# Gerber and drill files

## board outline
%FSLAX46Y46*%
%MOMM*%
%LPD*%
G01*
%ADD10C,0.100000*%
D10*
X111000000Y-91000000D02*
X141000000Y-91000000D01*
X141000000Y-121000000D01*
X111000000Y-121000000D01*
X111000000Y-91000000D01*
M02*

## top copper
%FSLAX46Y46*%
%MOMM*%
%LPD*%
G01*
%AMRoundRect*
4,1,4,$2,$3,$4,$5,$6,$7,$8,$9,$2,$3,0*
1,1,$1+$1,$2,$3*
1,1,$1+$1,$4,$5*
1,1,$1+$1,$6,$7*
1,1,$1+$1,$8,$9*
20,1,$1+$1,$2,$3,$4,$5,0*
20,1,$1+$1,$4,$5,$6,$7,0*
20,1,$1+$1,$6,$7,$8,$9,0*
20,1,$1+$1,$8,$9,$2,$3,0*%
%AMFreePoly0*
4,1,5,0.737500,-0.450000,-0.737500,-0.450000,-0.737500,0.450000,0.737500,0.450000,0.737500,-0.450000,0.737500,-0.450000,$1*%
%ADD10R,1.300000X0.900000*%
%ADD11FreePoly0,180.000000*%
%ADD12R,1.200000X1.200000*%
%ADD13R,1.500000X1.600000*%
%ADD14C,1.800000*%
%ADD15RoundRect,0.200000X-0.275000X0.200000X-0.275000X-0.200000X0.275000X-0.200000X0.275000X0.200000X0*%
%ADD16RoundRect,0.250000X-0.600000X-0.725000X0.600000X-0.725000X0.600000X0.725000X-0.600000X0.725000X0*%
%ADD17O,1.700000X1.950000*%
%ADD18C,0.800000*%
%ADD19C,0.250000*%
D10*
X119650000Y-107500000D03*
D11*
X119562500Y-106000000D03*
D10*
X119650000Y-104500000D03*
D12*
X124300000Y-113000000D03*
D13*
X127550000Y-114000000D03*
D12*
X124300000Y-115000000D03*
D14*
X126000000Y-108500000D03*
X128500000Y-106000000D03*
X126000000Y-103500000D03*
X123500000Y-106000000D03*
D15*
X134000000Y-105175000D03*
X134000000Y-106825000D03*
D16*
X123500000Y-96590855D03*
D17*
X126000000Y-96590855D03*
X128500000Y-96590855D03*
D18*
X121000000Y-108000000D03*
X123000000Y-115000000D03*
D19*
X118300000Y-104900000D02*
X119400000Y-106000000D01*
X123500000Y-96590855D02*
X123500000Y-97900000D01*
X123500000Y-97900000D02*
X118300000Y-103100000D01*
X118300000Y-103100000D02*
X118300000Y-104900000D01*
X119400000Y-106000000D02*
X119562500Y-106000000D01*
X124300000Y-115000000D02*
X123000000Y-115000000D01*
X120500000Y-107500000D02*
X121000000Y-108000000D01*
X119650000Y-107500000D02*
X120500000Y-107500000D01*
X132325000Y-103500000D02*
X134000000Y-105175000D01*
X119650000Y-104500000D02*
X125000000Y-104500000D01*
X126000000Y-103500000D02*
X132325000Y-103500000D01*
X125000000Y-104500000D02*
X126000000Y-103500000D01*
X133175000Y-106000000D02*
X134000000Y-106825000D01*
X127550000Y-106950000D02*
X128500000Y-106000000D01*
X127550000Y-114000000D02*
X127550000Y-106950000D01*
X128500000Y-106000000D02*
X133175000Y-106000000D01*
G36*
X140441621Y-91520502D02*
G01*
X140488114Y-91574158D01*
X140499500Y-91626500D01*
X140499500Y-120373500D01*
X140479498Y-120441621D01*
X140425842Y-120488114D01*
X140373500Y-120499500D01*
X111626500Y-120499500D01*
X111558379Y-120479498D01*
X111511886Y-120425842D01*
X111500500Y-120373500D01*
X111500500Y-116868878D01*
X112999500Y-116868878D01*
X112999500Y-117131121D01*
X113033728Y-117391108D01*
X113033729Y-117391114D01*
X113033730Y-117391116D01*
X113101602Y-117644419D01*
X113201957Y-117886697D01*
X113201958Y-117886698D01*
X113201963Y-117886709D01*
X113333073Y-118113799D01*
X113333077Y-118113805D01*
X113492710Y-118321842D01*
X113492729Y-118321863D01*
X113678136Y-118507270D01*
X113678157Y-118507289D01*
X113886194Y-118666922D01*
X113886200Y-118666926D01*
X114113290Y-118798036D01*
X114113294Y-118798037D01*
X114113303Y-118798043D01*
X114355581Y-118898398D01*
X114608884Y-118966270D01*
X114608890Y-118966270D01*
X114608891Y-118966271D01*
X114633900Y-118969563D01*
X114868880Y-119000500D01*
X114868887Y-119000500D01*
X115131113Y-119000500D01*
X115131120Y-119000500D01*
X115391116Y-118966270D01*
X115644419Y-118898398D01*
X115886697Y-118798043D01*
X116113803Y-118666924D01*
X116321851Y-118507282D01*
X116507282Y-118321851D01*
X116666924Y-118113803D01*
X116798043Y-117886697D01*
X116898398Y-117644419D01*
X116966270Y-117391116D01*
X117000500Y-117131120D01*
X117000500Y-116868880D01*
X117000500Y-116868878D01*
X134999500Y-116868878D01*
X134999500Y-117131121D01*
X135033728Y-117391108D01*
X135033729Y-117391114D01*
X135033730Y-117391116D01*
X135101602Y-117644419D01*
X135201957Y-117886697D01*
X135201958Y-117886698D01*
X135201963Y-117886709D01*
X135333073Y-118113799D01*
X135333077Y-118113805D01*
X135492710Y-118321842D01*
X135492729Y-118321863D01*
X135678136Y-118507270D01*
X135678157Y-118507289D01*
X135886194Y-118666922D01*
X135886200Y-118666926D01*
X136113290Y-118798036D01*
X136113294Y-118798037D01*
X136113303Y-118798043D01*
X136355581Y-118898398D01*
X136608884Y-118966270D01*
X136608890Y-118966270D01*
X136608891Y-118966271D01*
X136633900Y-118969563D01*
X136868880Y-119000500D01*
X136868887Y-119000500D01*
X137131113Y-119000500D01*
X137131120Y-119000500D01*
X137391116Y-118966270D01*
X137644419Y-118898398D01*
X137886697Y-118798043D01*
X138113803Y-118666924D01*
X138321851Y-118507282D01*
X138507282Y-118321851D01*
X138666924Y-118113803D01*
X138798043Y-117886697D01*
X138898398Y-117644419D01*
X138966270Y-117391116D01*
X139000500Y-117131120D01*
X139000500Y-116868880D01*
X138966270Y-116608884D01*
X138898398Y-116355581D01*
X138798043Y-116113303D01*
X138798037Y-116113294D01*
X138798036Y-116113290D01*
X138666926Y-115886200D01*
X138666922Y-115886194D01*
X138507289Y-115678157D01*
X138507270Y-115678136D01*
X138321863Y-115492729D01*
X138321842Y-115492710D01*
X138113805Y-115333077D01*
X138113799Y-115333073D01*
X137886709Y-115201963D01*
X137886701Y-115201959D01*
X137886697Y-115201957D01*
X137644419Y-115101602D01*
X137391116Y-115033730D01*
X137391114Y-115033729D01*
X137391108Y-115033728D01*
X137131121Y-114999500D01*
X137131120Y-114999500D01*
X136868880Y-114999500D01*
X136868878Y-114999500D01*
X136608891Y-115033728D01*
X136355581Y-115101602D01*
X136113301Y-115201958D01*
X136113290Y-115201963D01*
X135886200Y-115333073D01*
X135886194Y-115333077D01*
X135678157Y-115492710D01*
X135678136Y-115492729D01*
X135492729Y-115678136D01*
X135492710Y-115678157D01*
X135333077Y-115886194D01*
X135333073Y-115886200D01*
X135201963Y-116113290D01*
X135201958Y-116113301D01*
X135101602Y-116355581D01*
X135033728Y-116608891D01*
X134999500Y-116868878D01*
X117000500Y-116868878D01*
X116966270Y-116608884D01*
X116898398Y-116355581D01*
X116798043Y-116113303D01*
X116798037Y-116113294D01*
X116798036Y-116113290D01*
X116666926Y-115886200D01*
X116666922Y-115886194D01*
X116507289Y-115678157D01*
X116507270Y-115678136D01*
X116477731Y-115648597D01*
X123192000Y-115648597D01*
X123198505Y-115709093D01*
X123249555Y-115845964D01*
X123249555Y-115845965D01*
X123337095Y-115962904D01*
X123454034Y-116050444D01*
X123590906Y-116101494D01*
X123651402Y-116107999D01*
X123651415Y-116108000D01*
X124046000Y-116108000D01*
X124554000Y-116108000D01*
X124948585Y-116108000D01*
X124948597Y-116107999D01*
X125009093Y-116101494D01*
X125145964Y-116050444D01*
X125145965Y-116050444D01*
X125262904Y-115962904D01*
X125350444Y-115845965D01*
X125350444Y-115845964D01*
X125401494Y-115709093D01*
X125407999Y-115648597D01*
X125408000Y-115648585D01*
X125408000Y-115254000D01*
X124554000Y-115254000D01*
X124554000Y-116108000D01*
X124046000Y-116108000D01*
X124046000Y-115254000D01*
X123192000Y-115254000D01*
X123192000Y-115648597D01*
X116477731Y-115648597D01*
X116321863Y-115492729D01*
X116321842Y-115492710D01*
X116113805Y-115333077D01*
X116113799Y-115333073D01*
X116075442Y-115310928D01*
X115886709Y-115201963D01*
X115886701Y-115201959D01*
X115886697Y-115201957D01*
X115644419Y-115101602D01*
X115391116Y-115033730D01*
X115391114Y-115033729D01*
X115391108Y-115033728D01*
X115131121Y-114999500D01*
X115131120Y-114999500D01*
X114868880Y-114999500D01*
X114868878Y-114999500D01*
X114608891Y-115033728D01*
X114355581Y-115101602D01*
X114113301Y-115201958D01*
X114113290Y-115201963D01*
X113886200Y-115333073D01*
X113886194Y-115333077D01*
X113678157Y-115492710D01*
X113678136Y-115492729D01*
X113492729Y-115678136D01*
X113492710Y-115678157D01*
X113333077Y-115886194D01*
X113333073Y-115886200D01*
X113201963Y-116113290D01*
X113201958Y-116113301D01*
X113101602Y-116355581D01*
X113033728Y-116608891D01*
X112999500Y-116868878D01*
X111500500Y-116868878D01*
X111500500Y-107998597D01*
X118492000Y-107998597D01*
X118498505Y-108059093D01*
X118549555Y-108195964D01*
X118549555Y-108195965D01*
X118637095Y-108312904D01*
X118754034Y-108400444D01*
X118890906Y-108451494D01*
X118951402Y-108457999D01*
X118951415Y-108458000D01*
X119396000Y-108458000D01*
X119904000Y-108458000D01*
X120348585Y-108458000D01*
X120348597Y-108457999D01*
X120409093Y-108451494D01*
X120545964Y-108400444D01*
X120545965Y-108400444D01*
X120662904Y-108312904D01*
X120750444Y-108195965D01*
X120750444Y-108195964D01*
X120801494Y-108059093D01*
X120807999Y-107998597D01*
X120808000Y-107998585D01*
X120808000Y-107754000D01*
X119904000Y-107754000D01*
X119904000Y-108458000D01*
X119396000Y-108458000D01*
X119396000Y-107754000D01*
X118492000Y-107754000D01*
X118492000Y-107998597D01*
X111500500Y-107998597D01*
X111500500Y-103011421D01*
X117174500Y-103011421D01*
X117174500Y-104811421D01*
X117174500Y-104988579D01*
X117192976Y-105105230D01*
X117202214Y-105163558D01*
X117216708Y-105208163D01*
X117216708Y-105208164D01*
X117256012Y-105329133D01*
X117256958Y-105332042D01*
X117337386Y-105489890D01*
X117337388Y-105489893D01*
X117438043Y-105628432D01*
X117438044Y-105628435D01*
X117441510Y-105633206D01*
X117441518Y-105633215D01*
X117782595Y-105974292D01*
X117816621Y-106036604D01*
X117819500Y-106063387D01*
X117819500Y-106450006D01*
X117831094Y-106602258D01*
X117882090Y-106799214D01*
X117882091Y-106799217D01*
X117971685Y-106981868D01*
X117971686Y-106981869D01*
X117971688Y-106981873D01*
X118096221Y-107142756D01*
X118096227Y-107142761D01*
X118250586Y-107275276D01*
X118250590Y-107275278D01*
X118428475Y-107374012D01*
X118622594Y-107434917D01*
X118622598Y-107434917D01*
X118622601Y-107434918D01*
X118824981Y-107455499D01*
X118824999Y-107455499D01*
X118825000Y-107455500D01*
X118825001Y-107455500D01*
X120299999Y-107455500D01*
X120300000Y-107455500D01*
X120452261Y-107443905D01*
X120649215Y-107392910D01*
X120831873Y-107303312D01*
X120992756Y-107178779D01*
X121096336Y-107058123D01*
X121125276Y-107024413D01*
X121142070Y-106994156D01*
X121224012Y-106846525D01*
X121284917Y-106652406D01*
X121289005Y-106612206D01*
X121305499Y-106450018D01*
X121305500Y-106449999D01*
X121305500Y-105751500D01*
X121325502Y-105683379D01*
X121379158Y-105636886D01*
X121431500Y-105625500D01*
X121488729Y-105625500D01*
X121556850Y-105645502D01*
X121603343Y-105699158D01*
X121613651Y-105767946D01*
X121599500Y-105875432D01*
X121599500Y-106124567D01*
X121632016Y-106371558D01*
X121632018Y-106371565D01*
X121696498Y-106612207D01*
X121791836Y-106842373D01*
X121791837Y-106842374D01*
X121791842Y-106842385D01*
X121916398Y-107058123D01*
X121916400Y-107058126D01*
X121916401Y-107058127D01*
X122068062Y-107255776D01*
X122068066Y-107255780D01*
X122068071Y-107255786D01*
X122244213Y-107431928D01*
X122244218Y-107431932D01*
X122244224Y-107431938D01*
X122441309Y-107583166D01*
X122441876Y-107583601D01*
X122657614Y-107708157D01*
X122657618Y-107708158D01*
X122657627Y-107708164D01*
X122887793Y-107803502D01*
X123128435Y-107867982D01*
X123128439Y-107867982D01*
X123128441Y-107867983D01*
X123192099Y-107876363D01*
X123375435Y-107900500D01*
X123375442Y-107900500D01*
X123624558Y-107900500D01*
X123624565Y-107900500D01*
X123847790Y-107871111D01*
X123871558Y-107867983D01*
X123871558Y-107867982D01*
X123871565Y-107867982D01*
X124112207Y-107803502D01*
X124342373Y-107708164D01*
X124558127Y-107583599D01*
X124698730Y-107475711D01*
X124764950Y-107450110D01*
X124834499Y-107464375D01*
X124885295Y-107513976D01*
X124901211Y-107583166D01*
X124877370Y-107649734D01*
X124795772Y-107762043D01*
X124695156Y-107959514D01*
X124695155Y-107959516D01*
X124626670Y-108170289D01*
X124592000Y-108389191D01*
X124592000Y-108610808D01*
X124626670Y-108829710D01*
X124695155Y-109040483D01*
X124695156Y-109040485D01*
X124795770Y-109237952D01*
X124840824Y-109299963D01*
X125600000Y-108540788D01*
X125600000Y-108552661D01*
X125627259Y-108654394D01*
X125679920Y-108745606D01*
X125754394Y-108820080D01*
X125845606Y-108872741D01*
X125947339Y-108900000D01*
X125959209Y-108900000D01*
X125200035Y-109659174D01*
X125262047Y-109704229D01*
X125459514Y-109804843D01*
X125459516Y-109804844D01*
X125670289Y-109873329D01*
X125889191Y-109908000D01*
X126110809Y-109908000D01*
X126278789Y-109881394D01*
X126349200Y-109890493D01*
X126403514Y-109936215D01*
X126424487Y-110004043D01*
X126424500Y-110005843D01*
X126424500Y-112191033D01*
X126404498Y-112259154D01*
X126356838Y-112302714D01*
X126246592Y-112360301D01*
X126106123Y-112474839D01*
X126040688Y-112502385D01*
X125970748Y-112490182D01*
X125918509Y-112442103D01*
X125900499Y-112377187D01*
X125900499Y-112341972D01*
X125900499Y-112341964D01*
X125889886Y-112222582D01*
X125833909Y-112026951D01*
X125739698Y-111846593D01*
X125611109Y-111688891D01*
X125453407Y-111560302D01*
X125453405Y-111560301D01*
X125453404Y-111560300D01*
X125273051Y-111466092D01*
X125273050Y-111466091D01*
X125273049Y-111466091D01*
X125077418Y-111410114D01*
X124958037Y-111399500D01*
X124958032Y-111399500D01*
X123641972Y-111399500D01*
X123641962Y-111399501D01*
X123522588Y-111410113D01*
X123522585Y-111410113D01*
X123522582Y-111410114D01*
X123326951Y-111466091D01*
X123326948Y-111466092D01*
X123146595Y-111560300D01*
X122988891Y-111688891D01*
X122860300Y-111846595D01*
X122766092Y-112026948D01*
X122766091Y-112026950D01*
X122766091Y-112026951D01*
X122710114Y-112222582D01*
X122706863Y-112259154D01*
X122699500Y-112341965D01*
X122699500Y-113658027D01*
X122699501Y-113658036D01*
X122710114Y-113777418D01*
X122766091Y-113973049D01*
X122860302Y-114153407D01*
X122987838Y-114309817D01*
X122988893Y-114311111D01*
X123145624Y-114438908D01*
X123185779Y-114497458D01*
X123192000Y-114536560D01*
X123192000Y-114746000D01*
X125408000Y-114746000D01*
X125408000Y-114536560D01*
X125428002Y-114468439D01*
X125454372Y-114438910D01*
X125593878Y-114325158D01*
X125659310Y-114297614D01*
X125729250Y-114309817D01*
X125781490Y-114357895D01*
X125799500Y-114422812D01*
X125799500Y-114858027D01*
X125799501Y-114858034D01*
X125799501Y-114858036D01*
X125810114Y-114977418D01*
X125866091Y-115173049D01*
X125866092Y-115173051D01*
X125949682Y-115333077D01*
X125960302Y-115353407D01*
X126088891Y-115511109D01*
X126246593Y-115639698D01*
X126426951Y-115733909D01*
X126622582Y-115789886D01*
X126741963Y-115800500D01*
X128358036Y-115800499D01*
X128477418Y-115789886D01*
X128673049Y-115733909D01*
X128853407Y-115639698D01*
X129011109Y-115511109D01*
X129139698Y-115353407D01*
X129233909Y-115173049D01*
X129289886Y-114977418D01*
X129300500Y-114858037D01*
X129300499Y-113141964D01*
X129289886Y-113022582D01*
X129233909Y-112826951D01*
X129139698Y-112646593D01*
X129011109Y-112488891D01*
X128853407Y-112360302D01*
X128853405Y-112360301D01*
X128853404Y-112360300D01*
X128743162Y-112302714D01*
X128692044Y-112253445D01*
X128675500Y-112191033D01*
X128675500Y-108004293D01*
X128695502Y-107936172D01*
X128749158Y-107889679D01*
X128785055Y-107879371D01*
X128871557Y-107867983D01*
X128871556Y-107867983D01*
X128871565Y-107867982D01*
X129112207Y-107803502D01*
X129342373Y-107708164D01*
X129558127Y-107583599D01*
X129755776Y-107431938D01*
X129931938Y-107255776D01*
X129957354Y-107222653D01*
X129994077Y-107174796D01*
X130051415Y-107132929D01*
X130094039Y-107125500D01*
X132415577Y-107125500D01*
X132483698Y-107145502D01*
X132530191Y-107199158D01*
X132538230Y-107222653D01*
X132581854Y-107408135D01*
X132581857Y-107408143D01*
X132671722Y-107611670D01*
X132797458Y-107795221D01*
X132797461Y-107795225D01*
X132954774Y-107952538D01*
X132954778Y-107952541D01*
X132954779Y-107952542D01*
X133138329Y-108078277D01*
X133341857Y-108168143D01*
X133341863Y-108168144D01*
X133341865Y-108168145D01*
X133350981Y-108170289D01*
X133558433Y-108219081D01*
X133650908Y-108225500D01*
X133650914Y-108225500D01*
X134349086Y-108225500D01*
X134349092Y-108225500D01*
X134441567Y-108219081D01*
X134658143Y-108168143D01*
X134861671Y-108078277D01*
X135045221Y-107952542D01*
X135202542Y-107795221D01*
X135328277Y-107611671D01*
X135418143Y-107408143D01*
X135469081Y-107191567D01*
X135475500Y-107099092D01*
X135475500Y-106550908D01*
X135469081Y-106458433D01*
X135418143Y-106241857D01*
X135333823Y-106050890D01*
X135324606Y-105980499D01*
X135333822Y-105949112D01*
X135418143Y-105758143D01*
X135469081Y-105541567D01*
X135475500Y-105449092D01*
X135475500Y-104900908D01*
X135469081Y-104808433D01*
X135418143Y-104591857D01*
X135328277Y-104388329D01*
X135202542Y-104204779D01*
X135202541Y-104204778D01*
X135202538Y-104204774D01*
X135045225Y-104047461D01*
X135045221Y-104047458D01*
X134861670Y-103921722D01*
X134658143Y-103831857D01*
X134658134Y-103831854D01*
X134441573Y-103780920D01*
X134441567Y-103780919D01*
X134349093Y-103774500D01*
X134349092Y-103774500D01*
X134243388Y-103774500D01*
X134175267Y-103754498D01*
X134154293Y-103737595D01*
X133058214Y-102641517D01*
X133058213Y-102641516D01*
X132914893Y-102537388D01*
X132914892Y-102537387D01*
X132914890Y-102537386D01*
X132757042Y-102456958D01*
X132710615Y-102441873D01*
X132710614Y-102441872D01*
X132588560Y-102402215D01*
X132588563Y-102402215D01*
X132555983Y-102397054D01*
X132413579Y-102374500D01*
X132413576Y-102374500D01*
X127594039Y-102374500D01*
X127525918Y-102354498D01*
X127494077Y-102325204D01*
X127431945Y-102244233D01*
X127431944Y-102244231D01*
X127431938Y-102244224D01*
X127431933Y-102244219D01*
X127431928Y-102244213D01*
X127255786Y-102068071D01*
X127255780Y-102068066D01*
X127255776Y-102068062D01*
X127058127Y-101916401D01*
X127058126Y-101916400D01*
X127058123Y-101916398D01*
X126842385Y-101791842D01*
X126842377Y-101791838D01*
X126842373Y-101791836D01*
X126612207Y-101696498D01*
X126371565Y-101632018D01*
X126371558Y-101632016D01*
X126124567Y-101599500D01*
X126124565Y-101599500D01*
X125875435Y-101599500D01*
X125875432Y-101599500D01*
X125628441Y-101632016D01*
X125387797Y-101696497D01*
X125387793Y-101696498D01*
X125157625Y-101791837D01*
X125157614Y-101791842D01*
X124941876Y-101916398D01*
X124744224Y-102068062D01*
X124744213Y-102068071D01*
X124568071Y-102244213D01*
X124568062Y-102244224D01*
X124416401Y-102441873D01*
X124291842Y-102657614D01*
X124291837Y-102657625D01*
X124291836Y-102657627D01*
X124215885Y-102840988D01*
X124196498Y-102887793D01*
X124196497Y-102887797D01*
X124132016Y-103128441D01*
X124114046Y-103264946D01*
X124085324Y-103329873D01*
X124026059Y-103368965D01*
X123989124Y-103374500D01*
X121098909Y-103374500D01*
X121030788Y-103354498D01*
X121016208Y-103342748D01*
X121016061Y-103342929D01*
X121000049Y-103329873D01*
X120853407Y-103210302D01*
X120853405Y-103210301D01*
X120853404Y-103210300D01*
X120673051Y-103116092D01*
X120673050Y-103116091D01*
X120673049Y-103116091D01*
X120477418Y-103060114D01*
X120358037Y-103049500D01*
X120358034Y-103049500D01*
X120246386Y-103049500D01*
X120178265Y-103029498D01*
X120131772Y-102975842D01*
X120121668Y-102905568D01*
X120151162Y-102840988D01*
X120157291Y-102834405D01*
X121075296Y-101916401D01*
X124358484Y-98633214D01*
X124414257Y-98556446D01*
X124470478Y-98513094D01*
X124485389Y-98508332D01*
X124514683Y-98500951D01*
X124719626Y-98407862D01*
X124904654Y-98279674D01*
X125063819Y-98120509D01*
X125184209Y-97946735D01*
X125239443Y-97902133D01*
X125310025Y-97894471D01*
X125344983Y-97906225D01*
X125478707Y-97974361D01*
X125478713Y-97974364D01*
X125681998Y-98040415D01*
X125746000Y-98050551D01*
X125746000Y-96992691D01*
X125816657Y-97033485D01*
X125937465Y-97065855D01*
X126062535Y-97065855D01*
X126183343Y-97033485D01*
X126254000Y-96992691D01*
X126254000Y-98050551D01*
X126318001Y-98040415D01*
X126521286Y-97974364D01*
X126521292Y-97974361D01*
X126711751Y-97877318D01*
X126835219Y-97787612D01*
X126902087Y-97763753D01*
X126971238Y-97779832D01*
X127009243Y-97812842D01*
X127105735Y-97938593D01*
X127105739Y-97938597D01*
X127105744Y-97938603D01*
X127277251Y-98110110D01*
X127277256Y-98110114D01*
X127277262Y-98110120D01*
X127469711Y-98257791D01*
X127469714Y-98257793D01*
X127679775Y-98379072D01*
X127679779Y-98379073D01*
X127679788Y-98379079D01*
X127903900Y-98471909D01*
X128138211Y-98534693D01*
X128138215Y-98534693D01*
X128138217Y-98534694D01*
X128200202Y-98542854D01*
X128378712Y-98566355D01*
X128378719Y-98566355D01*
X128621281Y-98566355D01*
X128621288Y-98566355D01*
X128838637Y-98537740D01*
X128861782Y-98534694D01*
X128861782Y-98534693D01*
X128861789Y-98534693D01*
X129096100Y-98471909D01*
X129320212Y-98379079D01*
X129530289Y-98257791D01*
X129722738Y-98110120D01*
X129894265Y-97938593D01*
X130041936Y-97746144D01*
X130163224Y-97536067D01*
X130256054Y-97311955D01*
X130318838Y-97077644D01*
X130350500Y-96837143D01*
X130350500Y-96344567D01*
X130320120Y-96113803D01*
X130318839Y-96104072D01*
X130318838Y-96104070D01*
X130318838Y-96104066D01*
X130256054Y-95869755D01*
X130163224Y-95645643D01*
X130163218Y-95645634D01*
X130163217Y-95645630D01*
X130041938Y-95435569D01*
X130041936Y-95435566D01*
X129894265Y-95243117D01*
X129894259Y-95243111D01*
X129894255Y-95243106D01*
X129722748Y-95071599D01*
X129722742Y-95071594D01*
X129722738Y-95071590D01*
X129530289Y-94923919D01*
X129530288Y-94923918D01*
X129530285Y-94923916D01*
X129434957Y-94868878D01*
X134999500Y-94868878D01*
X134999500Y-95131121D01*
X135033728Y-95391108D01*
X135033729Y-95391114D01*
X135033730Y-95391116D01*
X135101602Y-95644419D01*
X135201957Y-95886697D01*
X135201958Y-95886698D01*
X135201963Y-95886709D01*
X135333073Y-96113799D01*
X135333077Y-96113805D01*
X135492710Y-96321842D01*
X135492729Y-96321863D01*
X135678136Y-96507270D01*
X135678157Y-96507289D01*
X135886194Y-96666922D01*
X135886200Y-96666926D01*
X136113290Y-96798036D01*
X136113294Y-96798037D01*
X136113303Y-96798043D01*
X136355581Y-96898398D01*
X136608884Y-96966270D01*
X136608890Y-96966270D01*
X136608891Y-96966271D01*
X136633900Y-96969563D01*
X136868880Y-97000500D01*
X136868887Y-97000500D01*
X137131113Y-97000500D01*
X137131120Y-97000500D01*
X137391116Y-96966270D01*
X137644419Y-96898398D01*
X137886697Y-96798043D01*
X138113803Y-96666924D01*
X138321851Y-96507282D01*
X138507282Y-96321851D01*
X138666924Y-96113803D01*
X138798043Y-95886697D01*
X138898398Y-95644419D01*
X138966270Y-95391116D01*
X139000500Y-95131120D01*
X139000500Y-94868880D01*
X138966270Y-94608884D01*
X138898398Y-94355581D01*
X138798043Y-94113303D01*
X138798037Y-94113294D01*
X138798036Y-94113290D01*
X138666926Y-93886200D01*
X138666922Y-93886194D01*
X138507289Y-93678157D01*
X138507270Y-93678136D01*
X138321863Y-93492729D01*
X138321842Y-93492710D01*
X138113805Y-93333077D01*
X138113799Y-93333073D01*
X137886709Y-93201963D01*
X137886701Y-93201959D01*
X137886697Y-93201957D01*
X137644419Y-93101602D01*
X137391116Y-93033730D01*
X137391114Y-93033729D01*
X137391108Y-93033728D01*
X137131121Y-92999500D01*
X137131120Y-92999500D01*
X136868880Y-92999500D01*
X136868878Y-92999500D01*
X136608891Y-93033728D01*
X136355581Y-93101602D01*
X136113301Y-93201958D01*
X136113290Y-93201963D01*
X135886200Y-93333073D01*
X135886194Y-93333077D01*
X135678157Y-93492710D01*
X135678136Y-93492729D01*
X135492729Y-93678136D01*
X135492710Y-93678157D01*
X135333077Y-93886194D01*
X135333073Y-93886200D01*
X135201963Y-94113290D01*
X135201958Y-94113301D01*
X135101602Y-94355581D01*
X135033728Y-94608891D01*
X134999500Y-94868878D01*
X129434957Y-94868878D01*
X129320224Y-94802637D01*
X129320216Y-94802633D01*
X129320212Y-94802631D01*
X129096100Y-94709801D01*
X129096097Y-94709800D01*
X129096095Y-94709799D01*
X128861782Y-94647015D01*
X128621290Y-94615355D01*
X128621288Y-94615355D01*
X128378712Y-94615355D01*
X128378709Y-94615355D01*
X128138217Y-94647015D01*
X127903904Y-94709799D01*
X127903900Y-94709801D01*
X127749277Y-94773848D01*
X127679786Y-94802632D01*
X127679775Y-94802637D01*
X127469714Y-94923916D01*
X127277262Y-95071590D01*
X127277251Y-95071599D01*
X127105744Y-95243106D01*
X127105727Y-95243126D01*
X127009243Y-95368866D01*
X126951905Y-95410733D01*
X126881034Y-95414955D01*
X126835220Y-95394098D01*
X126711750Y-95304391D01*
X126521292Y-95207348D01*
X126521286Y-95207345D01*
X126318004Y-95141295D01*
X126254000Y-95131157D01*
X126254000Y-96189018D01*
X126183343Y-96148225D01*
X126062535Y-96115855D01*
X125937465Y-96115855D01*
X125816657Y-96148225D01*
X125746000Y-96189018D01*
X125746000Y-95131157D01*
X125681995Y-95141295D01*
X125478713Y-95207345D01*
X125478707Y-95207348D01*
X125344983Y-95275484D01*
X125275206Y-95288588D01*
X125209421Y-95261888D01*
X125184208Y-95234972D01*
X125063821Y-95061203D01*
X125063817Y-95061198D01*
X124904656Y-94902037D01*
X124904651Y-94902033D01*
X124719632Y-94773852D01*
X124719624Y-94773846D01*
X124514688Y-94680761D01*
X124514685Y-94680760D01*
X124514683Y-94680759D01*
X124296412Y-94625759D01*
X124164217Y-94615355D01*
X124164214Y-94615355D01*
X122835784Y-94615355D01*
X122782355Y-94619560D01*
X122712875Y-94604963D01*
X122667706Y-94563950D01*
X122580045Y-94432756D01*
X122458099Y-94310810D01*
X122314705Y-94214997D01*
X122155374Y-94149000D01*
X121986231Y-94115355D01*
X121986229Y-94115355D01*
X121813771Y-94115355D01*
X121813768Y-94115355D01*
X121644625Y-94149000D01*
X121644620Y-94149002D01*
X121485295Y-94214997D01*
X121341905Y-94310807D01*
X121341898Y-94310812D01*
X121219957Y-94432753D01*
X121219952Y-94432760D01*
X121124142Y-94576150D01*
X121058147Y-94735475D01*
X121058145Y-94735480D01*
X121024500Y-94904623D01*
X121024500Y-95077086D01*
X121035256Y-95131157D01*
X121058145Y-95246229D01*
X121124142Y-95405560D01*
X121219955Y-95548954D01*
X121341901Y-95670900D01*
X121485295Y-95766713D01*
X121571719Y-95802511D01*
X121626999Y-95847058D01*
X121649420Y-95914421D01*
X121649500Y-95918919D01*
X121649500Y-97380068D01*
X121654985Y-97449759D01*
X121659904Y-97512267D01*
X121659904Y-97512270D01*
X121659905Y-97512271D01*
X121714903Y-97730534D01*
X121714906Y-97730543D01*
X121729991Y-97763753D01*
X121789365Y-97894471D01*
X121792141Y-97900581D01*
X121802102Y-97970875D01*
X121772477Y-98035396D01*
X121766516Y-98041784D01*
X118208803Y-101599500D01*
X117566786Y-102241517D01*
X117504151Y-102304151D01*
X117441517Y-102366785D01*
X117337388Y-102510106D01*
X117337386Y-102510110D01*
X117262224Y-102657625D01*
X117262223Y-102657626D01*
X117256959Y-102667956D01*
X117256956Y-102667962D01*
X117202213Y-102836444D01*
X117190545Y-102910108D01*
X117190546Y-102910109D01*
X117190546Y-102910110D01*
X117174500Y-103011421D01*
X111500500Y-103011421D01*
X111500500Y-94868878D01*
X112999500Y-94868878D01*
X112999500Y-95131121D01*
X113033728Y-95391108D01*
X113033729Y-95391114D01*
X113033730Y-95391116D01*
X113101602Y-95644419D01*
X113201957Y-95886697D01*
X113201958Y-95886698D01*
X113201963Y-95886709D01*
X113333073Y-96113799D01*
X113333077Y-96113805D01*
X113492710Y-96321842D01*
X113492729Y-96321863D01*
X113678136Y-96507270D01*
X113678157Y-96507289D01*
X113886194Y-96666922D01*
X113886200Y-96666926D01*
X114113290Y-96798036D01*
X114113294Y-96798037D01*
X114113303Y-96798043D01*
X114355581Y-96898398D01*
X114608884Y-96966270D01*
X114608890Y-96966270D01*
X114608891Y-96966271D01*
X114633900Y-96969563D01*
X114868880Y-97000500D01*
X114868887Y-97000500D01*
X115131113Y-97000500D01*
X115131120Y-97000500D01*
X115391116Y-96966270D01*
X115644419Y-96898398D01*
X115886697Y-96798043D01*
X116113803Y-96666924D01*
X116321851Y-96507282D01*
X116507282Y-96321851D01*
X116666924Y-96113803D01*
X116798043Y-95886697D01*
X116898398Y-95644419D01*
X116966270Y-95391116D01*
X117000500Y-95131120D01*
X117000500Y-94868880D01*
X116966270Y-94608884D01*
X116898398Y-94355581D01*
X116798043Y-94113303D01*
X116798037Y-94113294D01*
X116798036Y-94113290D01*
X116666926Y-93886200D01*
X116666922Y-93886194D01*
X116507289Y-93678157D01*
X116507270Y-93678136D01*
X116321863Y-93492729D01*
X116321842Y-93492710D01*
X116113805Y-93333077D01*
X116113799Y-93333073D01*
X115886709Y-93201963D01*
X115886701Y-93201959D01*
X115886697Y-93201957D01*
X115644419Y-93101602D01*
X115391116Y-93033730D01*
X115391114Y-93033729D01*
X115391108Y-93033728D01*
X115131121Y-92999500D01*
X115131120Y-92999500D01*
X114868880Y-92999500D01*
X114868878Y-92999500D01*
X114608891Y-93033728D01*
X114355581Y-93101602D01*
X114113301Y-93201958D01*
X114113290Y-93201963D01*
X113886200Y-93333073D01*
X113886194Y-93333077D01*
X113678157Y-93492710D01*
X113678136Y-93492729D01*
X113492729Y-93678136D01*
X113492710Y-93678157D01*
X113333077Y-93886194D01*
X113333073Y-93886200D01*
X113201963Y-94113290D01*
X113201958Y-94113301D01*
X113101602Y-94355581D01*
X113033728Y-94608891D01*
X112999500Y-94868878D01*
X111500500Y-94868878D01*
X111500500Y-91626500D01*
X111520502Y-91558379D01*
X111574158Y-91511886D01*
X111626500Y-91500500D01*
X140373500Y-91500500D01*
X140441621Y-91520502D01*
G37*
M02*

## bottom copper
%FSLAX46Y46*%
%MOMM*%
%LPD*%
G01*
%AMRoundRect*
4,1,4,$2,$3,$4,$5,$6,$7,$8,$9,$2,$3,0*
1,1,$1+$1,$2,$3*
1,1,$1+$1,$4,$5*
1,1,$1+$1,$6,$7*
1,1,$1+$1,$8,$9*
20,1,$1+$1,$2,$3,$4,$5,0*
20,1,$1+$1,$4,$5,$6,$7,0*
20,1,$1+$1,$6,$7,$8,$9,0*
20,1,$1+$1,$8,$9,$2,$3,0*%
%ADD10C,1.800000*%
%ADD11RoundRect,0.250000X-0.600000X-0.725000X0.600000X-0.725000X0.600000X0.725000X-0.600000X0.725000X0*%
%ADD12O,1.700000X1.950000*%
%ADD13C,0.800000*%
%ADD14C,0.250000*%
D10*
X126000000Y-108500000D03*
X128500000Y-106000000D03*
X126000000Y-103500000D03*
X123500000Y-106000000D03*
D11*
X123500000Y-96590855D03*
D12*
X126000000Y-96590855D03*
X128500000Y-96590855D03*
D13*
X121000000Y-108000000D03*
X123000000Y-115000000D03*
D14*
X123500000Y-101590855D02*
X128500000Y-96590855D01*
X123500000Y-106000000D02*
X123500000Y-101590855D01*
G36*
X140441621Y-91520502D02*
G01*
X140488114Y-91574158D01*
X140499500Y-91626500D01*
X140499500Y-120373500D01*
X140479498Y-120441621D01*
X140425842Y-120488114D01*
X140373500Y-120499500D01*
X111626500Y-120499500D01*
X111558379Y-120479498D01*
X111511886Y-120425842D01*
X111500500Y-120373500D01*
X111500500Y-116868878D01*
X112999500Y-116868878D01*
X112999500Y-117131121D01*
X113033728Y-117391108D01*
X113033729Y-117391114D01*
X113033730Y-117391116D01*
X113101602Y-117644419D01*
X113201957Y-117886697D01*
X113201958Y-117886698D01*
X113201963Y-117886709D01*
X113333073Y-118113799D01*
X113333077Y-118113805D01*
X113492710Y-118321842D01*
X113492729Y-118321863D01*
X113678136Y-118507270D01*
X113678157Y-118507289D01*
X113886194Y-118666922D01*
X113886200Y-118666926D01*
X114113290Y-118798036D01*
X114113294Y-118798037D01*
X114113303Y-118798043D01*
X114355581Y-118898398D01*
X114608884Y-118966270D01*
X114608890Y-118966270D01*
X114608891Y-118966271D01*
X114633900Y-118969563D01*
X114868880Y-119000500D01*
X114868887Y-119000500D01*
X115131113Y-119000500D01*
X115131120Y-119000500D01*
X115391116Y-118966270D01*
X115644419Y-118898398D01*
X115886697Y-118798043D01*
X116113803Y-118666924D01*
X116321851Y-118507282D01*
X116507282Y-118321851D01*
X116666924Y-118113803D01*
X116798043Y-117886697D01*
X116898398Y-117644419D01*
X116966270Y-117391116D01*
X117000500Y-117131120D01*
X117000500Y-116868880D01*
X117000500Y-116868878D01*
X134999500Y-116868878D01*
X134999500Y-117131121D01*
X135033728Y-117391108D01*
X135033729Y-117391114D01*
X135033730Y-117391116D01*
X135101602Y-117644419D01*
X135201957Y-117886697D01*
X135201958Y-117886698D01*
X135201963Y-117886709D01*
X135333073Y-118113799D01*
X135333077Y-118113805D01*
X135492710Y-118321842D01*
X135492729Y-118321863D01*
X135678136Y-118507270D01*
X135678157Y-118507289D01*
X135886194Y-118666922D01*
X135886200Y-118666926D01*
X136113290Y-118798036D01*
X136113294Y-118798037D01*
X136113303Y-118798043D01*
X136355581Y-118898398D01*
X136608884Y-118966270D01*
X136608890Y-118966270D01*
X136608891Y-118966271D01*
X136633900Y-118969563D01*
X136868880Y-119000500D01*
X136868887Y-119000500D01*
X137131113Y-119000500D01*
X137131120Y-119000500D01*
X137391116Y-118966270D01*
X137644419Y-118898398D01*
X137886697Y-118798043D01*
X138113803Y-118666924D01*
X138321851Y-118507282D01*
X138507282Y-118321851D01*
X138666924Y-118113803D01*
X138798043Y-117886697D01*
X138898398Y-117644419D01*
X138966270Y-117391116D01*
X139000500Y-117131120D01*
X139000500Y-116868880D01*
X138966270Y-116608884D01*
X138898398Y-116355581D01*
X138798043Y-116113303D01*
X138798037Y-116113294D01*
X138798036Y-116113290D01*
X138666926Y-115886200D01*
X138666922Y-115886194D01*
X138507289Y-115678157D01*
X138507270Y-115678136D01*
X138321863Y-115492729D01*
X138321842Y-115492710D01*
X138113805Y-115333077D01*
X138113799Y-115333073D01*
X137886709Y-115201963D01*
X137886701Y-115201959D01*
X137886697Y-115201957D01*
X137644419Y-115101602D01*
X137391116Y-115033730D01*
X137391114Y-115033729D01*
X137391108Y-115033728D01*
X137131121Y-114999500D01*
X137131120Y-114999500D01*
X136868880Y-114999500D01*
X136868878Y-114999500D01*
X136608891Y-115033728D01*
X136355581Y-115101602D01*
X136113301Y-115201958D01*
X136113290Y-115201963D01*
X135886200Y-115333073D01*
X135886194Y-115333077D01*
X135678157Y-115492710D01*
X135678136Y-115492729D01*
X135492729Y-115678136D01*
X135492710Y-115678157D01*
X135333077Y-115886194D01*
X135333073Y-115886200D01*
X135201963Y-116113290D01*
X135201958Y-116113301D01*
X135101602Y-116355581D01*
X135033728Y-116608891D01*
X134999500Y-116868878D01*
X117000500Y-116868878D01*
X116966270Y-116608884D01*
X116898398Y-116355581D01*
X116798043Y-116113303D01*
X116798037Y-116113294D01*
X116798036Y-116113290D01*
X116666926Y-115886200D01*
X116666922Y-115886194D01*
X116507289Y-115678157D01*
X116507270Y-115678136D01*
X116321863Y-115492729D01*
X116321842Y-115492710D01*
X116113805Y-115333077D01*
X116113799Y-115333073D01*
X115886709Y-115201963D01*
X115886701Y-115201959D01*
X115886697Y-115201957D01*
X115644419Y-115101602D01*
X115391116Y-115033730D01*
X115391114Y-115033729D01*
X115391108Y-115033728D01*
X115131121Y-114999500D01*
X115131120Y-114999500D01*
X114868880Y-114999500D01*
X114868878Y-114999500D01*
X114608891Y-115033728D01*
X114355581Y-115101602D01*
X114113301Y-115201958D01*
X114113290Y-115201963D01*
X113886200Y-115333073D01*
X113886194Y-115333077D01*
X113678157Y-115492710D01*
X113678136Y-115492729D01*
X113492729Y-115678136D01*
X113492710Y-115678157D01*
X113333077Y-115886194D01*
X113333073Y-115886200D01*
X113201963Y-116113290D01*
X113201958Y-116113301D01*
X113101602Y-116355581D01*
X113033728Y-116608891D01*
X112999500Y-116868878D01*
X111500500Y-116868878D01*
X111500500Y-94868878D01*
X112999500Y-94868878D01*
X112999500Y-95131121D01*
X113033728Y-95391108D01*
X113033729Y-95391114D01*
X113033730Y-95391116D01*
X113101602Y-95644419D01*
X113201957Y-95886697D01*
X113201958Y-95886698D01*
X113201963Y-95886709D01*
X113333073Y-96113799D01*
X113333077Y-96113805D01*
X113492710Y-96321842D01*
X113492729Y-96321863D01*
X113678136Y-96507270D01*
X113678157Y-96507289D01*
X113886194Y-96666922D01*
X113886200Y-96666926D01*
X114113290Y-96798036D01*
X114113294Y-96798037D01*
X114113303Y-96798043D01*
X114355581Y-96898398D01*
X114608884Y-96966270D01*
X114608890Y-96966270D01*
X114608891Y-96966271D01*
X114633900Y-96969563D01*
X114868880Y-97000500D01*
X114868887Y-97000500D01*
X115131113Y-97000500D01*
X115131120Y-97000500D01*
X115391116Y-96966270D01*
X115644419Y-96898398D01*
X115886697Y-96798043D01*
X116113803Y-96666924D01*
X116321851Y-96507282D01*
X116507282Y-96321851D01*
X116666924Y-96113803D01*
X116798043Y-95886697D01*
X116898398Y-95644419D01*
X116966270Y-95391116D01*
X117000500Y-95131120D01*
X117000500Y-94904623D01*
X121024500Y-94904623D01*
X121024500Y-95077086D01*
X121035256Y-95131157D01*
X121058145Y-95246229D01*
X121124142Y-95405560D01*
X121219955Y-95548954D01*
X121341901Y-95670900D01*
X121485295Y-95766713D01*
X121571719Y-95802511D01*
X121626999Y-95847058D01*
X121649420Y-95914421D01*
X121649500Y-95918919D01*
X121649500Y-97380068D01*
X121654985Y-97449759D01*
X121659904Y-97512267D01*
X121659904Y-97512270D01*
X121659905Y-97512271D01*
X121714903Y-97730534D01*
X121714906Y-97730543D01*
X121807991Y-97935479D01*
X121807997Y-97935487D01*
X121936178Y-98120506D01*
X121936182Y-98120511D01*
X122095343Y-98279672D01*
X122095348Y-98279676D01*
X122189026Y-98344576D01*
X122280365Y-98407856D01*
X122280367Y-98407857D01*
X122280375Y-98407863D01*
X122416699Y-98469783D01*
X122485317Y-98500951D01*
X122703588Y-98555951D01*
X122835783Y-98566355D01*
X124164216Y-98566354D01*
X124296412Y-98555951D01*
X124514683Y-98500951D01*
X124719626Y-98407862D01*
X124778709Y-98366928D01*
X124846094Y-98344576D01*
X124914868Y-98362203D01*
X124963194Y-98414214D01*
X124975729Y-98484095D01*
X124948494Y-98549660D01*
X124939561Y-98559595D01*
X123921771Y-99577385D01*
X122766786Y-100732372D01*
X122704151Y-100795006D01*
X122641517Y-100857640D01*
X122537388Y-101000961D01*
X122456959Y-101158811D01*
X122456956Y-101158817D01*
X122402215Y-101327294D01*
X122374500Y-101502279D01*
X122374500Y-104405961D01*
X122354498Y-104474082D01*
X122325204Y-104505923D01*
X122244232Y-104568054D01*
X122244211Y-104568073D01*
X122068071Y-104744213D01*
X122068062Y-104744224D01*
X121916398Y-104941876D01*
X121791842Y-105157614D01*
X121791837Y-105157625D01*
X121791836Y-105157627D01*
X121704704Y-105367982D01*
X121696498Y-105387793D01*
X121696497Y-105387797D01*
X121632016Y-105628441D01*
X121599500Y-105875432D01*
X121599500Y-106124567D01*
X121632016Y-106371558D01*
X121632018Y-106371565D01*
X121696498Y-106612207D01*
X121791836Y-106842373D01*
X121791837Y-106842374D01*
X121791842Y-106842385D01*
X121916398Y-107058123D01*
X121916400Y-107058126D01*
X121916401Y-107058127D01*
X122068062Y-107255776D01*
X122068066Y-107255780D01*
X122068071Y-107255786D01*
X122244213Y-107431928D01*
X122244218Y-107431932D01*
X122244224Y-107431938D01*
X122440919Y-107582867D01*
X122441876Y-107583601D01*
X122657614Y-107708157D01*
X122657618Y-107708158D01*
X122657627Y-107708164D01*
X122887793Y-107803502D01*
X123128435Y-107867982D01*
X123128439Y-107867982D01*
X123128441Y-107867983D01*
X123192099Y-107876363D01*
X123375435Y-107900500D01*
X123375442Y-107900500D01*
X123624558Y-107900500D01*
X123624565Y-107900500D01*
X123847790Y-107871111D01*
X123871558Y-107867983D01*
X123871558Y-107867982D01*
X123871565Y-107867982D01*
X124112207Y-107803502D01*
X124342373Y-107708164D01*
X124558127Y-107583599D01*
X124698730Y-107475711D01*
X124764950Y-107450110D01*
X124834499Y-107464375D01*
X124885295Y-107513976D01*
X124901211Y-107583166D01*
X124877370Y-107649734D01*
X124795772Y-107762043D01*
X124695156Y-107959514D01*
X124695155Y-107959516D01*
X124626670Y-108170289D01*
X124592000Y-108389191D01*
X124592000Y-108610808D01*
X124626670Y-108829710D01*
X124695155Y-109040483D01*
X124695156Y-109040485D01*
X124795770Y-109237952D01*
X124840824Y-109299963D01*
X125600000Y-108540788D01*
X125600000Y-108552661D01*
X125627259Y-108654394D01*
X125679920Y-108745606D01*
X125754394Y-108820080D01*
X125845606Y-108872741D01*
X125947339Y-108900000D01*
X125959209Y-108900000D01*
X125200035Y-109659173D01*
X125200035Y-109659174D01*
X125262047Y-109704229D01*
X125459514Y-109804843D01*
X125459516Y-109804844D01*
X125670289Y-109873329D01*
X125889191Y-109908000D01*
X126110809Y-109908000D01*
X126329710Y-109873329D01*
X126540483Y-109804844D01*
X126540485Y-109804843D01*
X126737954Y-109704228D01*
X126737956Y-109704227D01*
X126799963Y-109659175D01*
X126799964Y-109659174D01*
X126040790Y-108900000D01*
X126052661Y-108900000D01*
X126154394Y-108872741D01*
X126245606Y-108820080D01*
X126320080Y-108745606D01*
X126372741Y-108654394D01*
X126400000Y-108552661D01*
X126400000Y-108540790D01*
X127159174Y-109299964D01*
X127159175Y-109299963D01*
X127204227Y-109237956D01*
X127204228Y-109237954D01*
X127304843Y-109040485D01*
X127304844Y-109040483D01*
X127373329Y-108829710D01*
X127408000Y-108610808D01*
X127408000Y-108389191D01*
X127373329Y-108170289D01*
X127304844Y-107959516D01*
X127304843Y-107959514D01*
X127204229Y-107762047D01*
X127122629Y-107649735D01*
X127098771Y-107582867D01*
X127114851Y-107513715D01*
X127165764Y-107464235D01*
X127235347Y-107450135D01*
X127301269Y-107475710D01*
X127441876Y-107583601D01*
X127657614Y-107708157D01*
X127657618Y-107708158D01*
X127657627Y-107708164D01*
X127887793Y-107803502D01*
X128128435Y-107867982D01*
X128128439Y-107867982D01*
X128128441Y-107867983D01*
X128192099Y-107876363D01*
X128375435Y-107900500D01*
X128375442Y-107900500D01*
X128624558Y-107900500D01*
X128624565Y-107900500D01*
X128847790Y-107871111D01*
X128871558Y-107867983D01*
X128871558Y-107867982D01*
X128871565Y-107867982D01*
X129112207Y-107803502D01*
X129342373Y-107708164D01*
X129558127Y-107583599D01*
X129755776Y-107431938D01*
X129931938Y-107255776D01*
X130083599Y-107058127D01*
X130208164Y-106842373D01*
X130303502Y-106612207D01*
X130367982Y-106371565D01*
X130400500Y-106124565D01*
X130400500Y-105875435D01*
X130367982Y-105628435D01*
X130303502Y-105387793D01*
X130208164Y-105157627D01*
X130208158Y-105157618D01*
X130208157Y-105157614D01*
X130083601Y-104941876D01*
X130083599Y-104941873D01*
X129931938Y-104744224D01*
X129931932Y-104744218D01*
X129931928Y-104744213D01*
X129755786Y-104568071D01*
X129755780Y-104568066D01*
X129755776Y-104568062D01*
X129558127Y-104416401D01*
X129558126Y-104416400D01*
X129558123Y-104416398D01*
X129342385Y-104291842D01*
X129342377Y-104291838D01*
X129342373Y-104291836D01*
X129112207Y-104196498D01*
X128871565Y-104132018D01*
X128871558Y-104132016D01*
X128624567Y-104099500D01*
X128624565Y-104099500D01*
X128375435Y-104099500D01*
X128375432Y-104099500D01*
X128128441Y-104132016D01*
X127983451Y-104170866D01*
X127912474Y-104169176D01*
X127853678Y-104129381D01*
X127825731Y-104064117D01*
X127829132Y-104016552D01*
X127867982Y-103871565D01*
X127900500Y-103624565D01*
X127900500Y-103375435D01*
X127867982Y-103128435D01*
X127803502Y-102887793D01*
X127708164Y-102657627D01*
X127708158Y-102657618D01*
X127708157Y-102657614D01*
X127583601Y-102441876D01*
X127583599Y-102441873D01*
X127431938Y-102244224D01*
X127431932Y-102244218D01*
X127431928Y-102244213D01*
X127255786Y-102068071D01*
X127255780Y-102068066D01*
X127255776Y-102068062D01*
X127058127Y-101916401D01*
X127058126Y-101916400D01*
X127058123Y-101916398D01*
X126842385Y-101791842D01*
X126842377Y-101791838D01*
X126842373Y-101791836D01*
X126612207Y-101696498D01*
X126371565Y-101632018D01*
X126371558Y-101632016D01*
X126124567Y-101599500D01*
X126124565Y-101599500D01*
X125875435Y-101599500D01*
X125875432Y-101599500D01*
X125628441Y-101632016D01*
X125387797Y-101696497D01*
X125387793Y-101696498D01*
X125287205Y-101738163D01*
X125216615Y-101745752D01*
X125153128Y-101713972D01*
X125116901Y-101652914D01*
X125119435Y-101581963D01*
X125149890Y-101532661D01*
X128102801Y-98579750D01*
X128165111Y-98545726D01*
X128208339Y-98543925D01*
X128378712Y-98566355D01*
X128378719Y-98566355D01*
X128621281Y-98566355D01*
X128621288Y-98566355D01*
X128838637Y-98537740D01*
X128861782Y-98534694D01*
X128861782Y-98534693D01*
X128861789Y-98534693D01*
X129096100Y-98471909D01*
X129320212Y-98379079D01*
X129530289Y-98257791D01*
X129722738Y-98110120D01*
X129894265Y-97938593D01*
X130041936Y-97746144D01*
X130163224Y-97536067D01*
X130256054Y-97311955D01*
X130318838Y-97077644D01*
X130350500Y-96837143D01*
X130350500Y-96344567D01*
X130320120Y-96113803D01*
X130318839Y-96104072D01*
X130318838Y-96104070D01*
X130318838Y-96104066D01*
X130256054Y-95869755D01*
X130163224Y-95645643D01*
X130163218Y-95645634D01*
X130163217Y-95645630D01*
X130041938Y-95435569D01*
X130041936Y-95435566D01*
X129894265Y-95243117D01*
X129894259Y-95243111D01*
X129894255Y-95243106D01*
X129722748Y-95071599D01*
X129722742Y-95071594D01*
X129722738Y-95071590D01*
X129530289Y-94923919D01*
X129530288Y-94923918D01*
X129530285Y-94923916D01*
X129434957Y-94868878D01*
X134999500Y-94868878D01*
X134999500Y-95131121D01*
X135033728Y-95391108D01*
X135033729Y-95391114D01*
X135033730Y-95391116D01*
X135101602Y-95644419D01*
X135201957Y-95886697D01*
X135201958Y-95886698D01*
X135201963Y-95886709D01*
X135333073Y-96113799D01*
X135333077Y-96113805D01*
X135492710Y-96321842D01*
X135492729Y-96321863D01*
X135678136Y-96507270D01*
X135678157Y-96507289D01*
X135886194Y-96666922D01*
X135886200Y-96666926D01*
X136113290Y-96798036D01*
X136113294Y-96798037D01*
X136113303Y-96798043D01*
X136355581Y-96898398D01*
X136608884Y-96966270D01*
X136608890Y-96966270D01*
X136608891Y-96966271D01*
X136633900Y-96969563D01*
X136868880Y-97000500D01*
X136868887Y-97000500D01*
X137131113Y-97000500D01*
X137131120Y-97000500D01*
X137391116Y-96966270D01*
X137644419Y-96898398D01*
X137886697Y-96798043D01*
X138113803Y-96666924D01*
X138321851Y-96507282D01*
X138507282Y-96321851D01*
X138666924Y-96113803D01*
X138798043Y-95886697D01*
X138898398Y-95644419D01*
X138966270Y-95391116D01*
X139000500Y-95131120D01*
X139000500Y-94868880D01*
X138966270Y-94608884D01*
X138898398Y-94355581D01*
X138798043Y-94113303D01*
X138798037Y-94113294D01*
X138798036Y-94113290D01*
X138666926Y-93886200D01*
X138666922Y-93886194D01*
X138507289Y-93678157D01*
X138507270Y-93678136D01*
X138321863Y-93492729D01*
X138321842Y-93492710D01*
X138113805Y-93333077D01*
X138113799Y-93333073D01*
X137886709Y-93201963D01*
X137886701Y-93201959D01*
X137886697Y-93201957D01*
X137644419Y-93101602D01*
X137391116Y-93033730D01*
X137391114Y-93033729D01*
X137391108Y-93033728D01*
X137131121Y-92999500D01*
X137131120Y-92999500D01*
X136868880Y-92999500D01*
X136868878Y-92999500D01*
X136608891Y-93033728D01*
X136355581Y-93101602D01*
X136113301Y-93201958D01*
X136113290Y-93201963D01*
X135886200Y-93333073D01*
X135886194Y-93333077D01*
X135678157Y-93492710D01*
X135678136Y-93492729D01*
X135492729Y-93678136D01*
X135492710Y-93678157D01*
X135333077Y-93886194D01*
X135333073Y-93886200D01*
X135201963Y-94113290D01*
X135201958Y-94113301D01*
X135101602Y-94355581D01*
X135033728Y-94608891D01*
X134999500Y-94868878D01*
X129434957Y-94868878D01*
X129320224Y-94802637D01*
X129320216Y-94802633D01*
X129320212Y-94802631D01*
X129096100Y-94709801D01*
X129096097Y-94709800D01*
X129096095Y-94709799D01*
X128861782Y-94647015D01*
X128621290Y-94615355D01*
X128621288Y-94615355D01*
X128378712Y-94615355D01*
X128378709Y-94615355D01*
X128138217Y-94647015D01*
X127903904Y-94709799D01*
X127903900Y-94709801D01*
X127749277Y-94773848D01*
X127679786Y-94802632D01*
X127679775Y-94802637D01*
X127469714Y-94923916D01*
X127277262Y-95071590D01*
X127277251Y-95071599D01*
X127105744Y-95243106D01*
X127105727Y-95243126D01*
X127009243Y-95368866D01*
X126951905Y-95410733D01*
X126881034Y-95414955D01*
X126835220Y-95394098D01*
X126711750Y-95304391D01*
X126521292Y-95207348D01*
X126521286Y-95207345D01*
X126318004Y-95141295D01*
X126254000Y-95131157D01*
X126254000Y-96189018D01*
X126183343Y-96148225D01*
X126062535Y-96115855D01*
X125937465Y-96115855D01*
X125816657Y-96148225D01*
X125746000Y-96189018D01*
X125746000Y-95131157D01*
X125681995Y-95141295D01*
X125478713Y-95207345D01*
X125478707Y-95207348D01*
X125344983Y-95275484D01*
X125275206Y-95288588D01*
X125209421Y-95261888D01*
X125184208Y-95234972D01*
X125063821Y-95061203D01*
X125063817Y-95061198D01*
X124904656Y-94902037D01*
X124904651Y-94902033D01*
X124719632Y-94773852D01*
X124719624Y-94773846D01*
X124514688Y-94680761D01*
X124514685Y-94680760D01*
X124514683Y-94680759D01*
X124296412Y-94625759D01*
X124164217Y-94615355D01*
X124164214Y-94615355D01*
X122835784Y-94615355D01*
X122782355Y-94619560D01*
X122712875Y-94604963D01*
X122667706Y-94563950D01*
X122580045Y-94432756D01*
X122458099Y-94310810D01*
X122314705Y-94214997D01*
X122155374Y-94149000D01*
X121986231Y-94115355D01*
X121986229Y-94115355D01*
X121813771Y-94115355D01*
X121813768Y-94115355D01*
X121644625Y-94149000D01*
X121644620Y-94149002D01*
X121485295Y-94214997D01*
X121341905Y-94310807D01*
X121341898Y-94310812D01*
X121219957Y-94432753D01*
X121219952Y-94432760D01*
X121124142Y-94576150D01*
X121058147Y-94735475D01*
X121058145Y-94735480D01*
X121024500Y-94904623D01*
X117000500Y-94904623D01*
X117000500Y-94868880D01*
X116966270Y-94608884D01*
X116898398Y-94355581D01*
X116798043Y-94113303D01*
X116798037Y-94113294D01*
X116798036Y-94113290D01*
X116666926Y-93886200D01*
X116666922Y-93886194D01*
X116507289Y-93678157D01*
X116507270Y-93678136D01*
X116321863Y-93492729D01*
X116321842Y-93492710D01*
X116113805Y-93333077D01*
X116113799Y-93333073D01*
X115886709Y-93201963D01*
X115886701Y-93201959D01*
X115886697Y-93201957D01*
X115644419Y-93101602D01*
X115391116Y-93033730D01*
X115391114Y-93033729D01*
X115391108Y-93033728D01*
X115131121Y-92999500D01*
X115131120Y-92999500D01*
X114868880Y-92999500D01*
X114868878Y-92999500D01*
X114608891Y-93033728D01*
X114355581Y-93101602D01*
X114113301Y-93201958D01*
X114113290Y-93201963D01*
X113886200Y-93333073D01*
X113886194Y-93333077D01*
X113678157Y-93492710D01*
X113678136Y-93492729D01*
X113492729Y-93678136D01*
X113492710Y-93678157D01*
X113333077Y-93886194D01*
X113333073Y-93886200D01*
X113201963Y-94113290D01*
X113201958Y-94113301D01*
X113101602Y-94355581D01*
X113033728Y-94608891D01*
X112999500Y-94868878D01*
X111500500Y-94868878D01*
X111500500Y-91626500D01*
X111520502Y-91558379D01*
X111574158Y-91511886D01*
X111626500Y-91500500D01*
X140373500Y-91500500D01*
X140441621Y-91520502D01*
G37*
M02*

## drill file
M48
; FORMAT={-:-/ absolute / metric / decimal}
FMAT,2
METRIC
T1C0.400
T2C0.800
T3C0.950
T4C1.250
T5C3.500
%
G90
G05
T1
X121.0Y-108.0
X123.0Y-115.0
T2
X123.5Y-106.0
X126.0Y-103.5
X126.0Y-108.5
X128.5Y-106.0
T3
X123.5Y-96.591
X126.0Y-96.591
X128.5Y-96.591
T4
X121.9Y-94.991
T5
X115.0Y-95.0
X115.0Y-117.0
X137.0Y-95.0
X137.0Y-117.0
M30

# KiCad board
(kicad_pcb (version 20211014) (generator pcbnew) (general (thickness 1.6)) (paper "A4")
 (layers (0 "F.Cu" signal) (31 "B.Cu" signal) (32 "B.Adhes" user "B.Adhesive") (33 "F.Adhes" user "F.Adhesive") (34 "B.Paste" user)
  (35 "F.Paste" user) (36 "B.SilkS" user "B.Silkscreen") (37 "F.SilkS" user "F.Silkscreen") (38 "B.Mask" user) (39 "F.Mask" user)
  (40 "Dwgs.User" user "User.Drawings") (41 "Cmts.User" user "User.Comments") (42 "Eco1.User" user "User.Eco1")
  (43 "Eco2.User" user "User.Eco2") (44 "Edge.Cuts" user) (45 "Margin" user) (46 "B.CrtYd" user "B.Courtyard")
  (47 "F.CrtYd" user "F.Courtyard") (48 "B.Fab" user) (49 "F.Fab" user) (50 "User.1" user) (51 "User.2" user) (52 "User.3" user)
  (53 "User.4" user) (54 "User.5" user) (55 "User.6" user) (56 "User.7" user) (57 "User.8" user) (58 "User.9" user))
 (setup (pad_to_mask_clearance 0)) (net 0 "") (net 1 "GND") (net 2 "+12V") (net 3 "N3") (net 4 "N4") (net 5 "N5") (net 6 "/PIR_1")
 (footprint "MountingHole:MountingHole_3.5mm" (layer "F.Cu") (at 137 117)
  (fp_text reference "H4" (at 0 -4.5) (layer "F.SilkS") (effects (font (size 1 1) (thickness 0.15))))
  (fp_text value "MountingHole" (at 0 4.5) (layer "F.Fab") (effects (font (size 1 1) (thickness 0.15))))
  (pad "" np_thru_hole circle (at 0 0) (size 3.5 3.5) (drill 3.5) (layers *.Cu *.Mask)))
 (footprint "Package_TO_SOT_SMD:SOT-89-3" (layer "F.Cu") (at 118 106 180)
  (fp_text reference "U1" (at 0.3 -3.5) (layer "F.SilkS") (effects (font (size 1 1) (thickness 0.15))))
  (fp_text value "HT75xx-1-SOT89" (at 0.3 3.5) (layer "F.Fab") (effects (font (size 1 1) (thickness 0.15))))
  (pad "1" smd rect (at -1.65 -1.5 180) (size 1.3 0.9) (layers "F.Cu" "F.Paste" "F.Mask") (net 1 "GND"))
  (pad "2" smd custom (at -1.5625 0 180) (size 1.475 0.9) (layers "F.Cu" "F.Paste" "F.Mask") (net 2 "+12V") (zone_connect 2)
   (options (clearance outline) (anchor rect)) (primitives))
  (pad "3" smd rect (at -1.65 1.5 180) (size 1.3 0.9) (layers "F.Cu" "F.Paste" "F.Mask") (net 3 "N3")))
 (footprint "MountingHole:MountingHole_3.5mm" (layer "F.Cu") (at 137 95)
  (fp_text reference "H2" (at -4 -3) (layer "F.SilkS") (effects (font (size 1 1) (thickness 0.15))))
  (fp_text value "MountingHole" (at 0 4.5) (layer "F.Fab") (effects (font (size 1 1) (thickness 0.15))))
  (pad "" np_thru_hole circle (at 0 0) (size 3.5 3.5) (drill 3.5) (layers *.Cu *.Mask)))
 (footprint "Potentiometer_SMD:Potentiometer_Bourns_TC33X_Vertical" (layer "F.Cu") (at 126.1 114)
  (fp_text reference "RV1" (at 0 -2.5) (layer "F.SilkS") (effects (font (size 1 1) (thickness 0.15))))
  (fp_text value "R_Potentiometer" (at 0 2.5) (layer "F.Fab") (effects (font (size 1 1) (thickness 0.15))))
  (pad "1" smd rect (at -1.8 -1) (size 1.2 1.2) (layers "F.Cu" "F.Paste" "F.Mask") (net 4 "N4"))
  (pad "2" smd rect (at 1.45 0) (size 1.5 1.6) (layers "F.Cu" "F.Paste" "F.Mask") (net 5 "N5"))
  (pad "3" smd rect (at -1.8 1) (size 1.2 1.2) (layers "F.Cu" "F.Paste" "F.Mask") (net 1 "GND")))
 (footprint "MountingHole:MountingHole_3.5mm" (layer "F.Cu") (at 115 117)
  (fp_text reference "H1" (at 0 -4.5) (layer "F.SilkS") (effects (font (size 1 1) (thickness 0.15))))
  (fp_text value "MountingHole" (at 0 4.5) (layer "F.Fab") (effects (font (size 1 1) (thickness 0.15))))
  (pad "" np_thru_hole circle (at 0 0) (size 3.5 3.5) (drill 3.5) (layers *.Cu *.Mask)))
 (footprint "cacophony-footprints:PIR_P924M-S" (layer "F.Cu") (at 126 106)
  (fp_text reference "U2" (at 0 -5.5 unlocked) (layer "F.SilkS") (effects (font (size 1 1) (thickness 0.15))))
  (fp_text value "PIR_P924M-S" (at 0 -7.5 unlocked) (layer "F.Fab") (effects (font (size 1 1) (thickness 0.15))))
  (pad "1" thru_hole circle (at 0 2.5) (size 1.8 1.8) (drill 0.8) (layers *.Cu *.Mask) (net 1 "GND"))
  (pad "2" thru_hole circle (at 2.5 0) (size 1.8 1.8) (drill 0.8) (layers *.Cu *.Mask) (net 5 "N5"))
  (pad "3" thru_hole circle (at 0 -2.5) (size 1.8 1.8) (drill 0.8) (layers *.Cu *.Mask) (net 3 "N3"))
  (pad "4" thru_hole circle (at -2.5 0) (size 1.8 1.8) (drill 0.8) (layers *.Cu *.Mask) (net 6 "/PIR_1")))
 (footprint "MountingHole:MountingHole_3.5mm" (layer "F.Cu") (at 115 95)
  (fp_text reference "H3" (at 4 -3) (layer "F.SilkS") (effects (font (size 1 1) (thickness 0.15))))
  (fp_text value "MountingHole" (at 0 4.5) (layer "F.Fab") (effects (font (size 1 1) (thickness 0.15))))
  (pad "" np_thru_hole circle (at 0 0) (size 3.5 3.5) (drill 3.5) (layers *.Cu *.Mask)))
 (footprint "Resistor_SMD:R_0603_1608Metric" (layer "F.Cu") (at 134 106 -90)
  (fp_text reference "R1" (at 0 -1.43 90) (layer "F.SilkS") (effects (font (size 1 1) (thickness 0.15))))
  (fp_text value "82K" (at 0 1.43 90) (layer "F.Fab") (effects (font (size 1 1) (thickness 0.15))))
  (pad "1" smd roundrect (at -0.825 0 270) (size 0.8 0.95) (layers "F.Cu" "F.Paste" "F.Mask") (roundrect_rratio 0.25) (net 3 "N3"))
  (pad "2" smd roundrect (at 0.825 0 270) (size 0.8 0.95) (layers "F.Cu" "F.Paste" "F.Mask") (roundrect_rratio 0.25) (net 5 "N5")))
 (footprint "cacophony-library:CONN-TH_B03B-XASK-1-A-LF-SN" (layer "B.Cu") (at 126 96.6 180)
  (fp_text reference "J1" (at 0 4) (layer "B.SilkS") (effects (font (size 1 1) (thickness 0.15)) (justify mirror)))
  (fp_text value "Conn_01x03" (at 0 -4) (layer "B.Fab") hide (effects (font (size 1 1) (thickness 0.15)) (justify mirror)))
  (pad "" np_thru_hole circle (at 4.1 1.609145) (size 1.25 1.25) (drill 1.25) (layers *.Cu *.Mask))
  (pad "1" thru_hole roundrect (at 2.5 0.009145) (size 1.7 1.95) (drill 0.95) (layers *.Cu *.Mask) (roundrect_rratio 0.1470588235)
   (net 2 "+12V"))
  (pad "2" thru_hole oval (at 0 0.009145) (size 1.7 1.95) (drill 0.95) (layers *.Cu *.Mask) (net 1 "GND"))
  (pad "3" thru_hole oval (at -2.5 0.009145) (size 1.7 1.95) (drill 0.95) (layers *.Cu *.Mask) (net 6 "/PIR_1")))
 (gr_rect (start 111 121) (end 141 91) (layer "Edge.Cuts") (width 0.1) (fill none))
 (segment (start 118.3 104.9) (end 119.4 106) (width 0.25) (layer "F.Cu") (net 2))
 (segment (start 123.5 96.590855) (end 123.5 97.9) (width 0.25) (layer "F.Cu") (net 2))
 (segment (start 123.5 97.9) (end 118.3 103.1) (width 0.25) (layer "F.Cu") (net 2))
 (segment (start 118.3 103.1) (end 118.3 104.9) (width 0.25) (layer "F.Cu") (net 2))
 (segment (start 119.4 106) (end 119.5625 106) (width 0.25) (layer "F.Cu") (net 2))
 (segment (start 124.3 115) (end 123 115) (width 0.25) (layer "F.Cu") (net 1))
 (segment (start 120.5 107.5) (end 121 108) (width 0.25) (layer "F.Cu") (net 1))
 (segment (start 119.65 107.5) (end 120.5 107.5) (width 0.25) (layer "F.Cu") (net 1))
 (via (at 121 108) (size 0.8) (drill 0.4) (layers "F.Cu" "B.Cu") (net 1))
 (via (at 123 115) (size 0.8) (drill 0.4) (layers "F.Cu" "B.Cu") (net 1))
 (segment (start 123.5 101.590855) (end 128.5 96.590855) (width 0.25) (layer "B.Cu") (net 6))
 (segment (start 123.5 106) (end 123.5 101.590855) (width 0.25) (layer "B.Cu") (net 6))
 (segment (start 132.325 103.5) (end 134 105.175) (width 0.25) (layer "F.Cu") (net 3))
 (segment (start 119.65 104.5) (end 125 104.5) (width 0.25) (layer "F.Cu") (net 3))
 (segment (start 126 103.5) (end 132.325 103.5) (width 0.25) (layer "F.Cu") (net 3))
 (segment (start 125 104.5) (end 126 103.5) (width 0.25) (layer "F.Cu") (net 3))
 (segment (start 133.175 106) (end 134 106.825) (width 0.25) (layer "F.Cu") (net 5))
 (segment (start 127.55 106.95) (end 128.5 106) (width 0.25) (layer "F.Cu") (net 5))
 (segment (start 127.55 114) (end 127.55 106.95) (width 0.25) (layer "F.Cu") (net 5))
 (segment (start 128.5 106) (end 133.175 106) (width 0.25) (layer "F.Cu") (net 5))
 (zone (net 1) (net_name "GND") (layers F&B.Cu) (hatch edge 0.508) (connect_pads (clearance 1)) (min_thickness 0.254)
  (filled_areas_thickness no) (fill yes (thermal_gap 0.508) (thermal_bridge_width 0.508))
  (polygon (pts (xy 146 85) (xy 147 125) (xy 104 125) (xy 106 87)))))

